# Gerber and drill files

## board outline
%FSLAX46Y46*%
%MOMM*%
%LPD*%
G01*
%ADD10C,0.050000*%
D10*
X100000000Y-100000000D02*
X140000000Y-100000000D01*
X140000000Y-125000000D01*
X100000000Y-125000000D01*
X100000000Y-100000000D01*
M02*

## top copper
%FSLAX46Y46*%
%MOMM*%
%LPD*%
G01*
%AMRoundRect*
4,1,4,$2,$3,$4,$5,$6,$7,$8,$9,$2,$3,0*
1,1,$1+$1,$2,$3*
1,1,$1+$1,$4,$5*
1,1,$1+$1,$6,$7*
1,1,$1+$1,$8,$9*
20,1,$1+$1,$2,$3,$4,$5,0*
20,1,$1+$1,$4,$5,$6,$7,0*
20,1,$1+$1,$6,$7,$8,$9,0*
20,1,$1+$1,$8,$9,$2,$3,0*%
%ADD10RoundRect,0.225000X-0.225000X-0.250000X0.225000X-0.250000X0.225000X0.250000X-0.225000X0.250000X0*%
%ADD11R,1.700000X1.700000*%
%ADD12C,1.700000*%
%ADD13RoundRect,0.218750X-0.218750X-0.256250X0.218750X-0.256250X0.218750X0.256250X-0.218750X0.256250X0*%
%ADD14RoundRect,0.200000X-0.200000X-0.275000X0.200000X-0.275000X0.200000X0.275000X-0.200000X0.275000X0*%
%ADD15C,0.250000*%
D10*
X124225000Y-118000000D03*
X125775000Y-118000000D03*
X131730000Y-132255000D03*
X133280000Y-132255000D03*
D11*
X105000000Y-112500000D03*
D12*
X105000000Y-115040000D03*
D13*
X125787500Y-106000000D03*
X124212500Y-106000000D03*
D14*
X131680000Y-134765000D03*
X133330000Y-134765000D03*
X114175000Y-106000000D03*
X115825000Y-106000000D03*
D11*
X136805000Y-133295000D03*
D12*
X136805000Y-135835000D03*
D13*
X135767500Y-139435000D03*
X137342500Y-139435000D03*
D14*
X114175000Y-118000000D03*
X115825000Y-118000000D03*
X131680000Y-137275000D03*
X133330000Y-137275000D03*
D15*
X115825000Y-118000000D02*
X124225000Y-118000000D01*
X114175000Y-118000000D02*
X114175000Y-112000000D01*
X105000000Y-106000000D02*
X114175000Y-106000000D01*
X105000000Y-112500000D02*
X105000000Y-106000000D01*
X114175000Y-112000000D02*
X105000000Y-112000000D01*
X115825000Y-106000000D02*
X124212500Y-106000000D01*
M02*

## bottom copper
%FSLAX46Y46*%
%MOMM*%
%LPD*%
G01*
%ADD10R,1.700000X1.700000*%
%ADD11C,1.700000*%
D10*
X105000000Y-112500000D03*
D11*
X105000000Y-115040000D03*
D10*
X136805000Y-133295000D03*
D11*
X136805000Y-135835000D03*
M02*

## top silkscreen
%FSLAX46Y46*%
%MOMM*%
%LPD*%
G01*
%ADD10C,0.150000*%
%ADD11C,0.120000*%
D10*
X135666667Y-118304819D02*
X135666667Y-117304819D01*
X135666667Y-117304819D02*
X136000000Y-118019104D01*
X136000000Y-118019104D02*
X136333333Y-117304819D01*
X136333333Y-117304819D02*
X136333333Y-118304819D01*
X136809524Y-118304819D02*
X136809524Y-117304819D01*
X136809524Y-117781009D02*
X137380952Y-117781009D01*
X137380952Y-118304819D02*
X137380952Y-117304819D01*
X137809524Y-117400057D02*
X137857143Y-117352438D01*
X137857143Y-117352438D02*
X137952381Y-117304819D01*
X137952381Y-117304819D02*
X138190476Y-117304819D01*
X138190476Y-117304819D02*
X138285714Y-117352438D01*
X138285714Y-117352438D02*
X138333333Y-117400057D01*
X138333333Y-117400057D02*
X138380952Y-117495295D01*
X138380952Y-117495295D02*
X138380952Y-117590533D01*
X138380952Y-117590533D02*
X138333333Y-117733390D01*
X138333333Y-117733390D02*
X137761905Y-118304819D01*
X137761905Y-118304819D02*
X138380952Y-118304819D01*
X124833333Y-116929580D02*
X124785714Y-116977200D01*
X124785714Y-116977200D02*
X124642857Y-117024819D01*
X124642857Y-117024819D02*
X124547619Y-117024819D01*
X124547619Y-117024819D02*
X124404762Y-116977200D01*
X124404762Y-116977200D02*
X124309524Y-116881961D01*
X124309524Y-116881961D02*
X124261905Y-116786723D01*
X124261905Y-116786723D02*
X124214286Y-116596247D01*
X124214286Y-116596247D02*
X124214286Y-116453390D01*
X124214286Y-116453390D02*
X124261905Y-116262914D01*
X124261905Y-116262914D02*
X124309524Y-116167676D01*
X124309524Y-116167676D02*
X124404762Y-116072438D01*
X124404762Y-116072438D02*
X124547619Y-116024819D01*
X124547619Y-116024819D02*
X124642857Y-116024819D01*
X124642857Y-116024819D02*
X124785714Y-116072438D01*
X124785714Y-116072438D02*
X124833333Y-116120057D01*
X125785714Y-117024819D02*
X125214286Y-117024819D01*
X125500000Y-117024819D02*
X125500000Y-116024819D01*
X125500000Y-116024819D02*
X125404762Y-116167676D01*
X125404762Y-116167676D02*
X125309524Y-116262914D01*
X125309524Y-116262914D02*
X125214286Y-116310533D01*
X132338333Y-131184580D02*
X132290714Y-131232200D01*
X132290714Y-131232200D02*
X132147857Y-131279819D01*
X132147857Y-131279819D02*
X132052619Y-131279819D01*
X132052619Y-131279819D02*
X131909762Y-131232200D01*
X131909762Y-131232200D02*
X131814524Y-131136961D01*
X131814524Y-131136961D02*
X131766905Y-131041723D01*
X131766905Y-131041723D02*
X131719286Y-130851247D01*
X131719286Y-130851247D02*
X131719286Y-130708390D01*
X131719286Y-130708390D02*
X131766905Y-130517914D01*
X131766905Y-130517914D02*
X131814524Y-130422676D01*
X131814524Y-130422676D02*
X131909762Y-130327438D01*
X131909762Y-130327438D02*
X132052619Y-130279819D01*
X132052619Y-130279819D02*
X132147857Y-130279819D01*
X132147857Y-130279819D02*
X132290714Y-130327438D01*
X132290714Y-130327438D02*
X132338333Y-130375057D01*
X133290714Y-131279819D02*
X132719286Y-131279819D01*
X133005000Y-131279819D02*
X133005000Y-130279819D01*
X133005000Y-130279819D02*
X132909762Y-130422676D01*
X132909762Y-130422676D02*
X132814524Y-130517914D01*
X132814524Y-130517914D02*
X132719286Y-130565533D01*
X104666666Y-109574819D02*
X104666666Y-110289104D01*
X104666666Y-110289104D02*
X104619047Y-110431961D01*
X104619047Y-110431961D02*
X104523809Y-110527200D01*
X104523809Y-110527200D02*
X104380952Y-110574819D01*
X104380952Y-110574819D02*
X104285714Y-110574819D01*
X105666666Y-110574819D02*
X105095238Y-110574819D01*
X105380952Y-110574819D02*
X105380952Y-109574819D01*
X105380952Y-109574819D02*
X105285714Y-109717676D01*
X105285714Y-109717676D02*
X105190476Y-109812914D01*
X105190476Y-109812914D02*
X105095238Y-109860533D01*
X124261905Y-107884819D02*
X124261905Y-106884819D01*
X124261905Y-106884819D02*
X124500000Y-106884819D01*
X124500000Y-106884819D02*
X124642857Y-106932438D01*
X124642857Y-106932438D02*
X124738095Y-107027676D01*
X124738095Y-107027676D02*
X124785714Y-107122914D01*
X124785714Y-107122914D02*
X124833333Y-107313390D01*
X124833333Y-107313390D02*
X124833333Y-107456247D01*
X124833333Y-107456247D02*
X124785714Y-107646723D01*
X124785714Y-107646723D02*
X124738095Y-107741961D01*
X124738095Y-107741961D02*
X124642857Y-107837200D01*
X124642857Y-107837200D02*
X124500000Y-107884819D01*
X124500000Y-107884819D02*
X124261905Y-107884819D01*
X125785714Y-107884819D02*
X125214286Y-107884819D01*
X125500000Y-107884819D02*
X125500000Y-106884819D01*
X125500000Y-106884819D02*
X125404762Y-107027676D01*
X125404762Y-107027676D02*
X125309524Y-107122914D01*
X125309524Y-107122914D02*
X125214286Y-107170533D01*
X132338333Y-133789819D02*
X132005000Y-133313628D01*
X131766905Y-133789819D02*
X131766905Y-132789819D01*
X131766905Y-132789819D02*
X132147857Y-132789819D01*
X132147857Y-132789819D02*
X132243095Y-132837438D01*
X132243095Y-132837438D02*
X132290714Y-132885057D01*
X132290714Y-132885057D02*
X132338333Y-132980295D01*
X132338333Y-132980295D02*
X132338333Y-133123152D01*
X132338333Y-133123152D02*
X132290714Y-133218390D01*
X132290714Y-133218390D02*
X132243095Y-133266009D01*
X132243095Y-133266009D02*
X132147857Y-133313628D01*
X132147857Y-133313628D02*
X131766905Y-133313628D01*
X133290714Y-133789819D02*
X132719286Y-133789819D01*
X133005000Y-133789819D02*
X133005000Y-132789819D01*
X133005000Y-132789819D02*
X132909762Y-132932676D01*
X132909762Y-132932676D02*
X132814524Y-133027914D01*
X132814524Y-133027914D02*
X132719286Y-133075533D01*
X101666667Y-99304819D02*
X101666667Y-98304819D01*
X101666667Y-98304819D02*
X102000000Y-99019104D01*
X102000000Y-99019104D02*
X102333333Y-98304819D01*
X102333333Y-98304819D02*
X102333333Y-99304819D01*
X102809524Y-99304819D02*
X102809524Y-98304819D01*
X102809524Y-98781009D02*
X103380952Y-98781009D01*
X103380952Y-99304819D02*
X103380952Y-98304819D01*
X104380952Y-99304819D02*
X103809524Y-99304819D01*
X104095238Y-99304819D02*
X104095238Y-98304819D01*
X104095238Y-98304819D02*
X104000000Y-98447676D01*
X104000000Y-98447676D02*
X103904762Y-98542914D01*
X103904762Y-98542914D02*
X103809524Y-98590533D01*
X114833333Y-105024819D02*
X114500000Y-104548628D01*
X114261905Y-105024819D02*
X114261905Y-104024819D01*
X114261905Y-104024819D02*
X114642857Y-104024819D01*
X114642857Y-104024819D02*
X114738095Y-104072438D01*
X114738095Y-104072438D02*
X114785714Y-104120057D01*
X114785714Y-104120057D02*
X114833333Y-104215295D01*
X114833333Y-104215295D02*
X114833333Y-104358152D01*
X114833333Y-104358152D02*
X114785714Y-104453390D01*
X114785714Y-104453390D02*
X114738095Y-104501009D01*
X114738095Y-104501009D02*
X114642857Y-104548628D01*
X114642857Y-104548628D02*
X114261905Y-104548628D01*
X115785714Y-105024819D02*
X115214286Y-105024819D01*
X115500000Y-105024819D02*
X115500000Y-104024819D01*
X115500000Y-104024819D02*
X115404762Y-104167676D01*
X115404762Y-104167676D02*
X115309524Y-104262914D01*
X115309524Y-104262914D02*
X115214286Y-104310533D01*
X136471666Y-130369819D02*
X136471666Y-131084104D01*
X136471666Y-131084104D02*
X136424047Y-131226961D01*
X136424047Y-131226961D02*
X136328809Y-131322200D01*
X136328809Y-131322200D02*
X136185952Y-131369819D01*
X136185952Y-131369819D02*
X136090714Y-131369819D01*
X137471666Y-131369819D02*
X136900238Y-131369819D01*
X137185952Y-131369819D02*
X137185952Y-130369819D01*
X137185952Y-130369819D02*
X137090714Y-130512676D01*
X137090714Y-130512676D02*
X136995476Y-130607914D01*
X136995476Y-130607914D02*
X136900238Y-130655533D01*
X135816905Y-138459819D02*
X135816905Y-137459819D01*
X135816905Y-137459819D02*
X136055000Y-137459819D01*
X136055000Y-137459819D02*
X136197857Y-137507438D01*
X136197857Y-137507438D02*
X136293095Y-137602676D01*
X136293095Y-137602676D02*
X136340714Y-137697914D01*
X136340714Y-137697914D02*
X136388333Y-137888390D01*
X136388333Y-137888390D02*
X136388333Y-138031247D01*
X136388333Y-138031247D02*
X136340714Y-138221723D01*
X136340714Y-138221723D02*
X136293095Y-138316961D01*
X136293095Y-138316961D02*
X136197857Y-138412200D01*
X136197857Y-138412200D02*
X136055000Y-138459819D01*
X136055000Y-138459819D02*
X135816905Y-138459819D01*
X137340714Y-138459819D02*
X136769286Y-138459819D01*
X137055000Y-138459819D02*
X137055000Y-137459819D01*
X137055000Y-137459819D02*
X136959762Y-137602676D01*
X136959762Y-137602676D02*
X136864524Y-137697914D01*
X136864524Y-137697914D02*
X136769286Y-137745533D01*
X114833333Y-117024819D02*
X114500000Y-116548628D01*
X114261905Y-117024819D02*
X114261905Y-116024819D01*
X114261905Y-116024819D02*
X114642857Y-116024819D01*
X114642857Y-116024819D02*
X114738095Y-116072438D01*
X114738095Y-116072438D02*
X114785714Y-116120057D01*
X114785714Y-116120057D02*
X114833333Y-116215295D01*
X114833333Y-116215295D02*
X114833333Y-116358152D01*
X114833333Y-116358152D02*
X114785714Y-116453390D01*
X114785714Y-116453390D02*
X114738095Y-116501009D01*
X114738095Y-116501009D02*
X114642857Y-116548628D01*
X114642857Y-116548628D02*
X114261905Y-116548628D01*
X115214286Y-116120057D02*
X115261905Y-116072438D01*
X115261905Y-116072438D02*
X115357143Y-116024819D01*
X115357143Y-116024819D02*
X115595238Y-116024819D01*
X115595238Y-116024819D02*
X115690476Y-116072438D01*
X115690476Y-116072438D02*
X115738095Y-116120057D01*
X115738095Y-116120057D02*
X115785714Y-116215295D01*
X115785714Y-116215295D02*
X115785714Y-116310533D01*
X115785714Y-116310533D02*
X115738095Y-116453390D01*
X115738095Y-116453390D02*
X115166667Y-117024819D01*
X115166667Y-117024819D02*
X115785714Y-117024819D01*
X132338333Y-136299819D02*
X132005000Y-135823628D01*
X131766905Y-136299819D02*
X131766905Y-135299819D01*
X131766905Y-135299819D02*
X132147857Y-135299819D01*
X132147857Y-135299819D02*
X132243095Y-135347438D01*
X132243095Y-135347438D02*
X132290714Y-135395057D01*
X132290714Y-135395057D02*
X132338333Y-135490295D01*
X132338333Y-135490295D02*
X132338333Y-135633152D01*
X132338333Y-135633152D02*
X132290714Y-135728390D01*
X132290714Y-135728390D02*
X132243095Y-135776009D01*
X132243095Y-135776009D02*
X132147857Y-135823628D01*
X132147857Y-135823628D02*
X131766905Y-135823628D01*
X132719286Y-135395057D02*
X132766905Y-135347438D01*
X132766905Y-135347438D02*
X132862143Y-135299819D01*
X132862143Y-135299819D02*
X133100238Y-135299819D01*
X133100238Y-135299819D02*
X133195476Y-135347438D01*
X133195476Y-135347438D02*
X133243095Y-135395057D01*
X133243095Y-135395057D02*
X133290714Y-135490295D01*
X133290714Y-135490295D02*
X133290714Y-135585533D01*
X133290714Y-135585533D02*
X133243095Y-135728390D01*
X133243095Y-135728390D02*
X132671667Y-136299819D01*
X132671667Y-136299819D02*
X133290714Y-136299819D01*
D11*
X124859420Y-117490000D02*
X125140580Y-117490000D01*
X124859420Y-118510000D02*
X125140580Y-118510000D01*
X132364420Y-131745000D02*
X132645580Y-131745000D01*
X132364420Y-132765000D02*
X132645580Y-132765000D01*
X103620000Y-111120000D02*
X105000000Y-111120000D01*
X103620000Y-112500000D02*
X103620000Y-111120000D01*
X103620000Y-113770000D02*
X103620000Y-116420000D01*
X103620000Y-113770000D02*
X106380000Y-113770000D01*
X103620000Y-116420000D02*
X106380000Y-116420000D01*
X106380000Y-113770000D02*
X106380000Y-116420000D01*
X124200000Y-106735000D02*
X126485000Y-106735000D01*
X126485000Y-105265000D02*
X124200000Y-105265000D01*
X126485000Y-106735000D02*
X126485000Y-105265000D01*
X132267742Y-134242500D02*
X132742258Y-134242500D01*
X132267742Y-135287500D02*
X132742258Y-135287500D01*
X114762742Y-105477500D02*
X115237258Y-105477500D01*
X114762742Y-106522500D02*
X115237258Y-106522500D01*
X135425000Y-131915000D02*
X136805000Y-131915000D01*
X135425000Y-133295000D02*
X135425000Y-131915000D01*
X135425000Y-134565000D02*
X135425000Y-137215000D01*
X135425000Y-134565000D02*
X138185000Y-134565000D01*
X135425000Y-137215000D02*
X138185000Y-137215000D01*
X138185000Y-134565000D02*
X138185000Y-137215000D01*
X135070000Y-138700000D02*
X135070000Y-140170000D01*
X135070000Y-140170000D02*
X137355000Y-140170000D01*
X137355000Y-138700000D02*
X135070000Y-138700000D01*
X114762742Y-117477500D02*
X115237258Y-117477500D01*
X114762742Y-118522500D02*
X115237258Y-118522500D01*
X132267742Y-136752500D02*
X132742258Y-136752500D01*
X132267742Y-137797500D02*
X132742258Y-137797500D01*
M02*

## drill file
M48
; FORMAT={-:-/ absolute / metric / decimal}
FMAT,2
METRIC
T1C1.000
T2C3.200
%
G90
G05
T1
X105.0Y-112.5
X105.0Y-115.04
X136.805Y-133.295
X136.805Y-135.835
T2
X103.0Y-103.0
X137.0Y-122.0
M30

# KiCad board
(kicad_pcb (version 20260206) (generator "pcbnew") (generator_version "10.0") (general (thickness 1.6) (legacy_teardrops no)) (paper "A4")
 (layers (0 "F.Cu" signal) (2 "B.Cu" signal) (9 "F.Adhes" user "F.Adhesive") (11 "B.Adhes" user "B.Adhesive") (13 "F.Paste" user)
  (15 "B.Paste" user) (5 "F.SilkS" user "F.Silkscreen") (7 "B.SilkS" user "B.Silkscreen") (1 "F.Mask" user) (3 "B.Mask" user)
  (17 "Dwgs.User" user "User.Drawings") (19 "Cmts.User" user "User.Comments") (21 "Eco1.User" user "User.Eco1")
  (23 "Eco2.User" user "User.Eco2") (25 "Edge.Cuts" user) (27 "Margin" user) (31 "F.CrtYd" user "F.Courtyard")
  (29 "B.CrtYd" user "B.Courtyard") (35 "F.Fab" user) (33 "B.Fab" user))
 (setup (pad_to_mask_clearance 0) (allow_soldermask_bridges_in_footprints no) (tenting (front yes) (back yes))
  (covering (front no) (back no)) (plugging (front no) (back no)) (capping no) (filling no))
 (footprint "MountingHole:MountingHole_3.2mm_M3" (layer "F.Cu") (at 137 122)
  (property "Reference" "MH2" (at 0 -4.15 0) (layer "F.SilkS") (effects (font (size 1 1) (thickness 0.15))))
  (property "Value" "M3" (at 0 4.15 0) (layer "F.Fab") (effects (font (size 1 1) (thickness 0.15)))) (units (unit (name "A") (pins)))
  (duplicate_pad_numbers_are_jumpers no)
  (pad "" np_thru_hole circle (at 0 0) (size 3.2 3.2) (drill 3.2) (layers "*.Cu" "*.Mask")))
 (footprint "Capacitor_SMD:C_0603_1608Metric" (layer "F.Cu") (at 125 118)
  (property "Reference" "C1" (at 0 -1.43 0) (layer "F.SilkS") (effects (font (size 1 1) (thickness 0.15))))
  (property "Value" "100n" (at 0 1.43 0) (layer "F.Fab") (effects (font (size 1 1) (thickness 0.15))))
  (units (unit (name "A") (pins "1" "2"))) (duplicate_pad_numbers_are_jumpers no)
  (fp_line (start -0.14058 -0.51) (end 0.14058 -0.51) (stroke (width 0.12) (type solid)) (layer "F.SilkS"))
  (fp_line (start -0.14058 0.51) (end 0.14058 0.51) (stroke (width 0.12) (type solid)) (layer "F.SilkS"))
  (pad "1" smd roundrect (at -0.775 0) (size 0.9 0.95) (layers "F.Cu" "F.Mask" "F.Paste") (roundrect_rratio 0.25) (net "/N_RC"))
  (pad "2" smd roundrect (at 0.775 0) (size 0.9 0.95) (layers "F.Cu" "F.Mask" "F.Paste") (roundrect_rratio 0.25) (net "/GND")))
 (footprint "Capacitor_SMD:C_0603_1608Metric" (layer "F.Cu") (at 132.505 132.255)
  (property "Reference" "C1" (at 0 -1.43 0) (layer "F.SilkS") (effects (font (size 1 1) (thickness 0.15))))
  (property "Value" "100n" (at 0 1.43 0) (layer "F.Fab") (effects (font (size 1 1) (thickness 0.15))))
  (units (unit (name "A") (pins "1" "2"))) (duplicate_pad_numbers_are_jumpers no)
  (fp_line (start -0.14058 -0.51) (end 0.14058 -0.51) (stroke (width 0.12) (type solid)) (layer "F.SilkS"))
  (fp_line (start -0.14058 0.51) (end 0.14058 0.51) (stroke (width 0.12) (type solid)) (layer "F.SilkS"))
  (pad "1" smd roundrect (at -0.775 0) (size 0.9 0.95) (layers "F.Cu" "F.Mask" "F.Paste") (roundrect_rratio 0.25) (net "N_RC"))
  (pad "2" smd roundrect (at 0.775 0) (size 0.9 0.95) (layers "F.Cu" "F.Mask" "F.Paste") (roundrect_rratio 0.25) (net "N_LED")))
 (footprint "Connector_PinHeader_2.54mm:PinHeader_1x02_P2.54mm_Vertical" (layer "F.Cu") (at 105 112.5)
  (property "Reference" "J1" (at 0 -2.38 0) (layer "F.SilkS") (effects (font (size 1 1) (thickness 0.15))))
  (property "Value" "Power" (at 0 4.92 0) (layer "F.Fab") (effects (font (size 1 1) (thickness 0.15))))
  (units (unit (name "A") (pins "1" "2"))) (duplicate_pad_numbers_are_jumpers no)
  (fp_line (start -1.38 -1.38) (end 0 -1.38) (stroke (width 0.12) (type solid)) (layer "F.SilkS"))
  (fp_line (start -1.38 0) (end -1.38 -1.38) (stroke (width 0.12) (type solid)) (layer "F.SilkS"))
  (fp_line (start -1.38 1.27) (end -1.38 3.92) (stroke (width 0.12) (type solid)) (layer "F.SilkS"))
  (fp_line (start -1.38 1.27) (end 1.38 1.27) (stroke (width 0.12) (type solid)) (layer "F.SilkS"))
  (fp_line (start -1.38 3.92) (end 1.38 3.92) (stroke (width 0.12) (type solid)) (layer "F.SilkS"))
  (fp_line (start 1.38 1.27) (end 1.38 3.92) (stroke (width 0.12) (type solid)) (layer "F.SilkS"))
  (pad "1" thru_hole rect (at 0 0) (size 1.7 1.7) (drill 1) (layers "*.Cu" "*.Mask") (remove_unused_layers no) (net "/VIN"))
  (pad "2" thru_hole circle (at 0 2.54) (size 1.7 1.7) (drill 1) (layers "*.Cu" "*.Mask") (remove_unused_layers no) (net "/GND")))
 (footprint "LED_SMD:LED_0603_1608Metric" (layer "F.Cu") (at 125 106 180)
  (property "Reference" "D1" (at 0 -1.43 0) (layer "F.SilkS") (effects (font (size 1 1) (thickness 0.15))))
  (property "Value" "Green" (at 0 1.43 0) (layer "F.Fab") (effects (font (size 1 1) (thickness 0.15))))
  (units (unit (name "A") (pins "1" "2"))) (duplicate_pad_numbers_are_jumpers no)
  (fp_line (start 0.8 -0.735) (end -1.485 -0.735) (stroke (width 0.12) (type solid)) (layer "F.SilkS"))
  (fp_line (start -1.485 0.735) (end 0.8 0.735) (stroke (width 0.12) (type solid)) (layer "F.SilkS"))
  (fp_line (start -1.485 -0.735) (end -1.485 0.735) (stroke (width 0.12) (type solid)) (layer "F.SilkS"))
  (pad "1" smd roundrect (at -0.7875 0) (size 0.875 0.95) (layers "F.Cu" "F.Mask" "F.Paste") (roundrect_rratio 0.25) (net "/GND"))
  (pad "2" smd roundrect (at 0.7875 0) (size 0.875 0.95) (layers "F.Cu" "F.Mask" "F.Paste") (roundrect_rratio 0.25) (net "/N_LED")))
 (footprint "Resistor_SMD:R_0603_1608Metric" (layer "F.Cu") (at 132.505 134.765)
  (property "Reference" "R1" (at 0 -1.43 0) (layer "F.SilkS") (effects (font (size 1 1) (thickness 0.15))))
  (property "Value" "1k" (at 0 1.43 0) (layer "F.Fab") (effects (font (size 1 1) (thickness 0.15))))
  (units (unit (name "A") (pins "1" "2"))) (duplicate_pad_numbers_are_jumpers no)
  (fp_line (start -0.237258 -0.5225) (end 0.237258 -0.5225) (stroke (width 0.12) (type solid)) (layer "F.SilkS"))
  (fp_line (start -0.237258 0.5225) (end 0.237258 0.5225) (stroke (width 0.12) (type solid)) (layer "F.SilkS"))
  (pad "1" smd roundrect (at -0.825 0) (size 0.8 0.95) (layers "F.Cu" "F.Mask" "F.Paste") (roundrect_rratio 0.25) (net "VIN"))
  (pad "2" smd roundrect (at 0.825 0) (size 0.8 0.95) (layers "F.Cu" "F.Mask" "F.Paste") (roundrect_rratio 0.25) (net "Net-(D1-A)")))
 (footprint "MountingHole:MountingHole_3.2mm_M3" (layer "F.Cu") (at 103 103)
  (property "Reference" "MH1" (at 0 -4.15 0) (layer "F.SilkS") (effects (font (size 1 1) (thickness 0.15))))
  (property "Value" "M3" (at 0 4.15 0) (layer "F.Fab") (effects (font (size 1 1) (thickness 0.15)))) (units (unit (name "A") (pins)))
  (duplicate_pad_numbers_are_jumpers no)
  (pad "" np_thru_hole circle (at 0 0) (size 3.2 3.2) (drill 3.2) (layers "*.Cu" "*.Mask")))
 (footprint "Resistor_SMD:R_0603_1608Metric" (layer "F.Cu") (at 115 106)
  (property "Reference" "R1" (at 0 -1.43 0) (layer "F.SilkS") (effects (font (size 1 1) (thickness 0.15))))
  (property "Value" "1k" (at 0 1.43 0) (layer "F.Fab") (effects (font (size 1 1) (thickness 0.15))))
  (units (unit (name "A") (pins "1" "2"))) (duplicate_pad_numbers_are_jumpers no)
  (fp_line (start -0.237258 -0.5225) (end 0.237258 -0.5225) (stroke (width 0.12) (type solid)) (layer "F.SilkS"))
  (fp_line (start -0.237258 0.5225) (end 0.237258 0.5225) (stroke (width 0.12) (type solid)) (layer "F.SilkS"))
  (pad "1" smd roundrect (at -0.825 0) (size 0.8 0.95) (layers "F.Cu" "F.Mask" "F.Paste") (roundrect_rratio 0.25) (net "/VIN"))
  (pad "2" smd roundrect (at 0.825 0) (size 0.8 0.95) (layers "F.Cu" "F.Mask" "F.Paste") (roundrect_rratio 0.25) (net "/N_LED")))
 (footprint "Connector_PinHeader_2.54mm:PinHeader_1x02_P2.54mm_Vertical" (layer "F.Cu") (at 136.805 133.295)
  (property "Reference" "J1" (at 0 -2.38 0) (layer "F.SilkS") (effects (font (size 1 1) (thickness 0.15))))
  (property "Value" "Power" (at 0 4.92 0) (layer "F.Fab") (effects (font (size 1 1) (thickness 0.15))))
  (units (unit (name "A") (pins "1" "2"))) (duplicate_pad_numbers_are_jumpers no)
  (fp_line (start -1.38 -1.38) (end 0 -1.38) (stroke (width 0.12) (type solid)) (layer "F.SilkS"))
  (fp_line (start -1.38 0) (end -1.38 -1.38) (stroke (width 0.12) (type solid)) (layer "F.SilkS"))
  (fp_line (start -1.38 1.27) (end -1.38 3.92) (stroke (width 0.12) (type solid)) (layer "F.SilkS"))
  (fp_line (start -1.38 1.27) (end 1.38 1.27) (stroke (width 0.12) (type solid)) (layer "F.SilkS"))
  (fp_line (start -1.38 3.92) (end 1.38 3.92) (stroke (width 0.12) (type solid)) (layer "F.SilkS"))
  (fp_line (start 1.38 1.27) (end 1.38 3.92) (stroke (width 0.12) (type solid)) (layer "F.SilkS"))
  (pad "1" thru_hole rect (at 0 0) (size 1.7 1.7) (drill 1) (layers "*.Cu" "*.Mask") (remove_unused_layers no) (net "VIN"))
  (pad "2" thru_hole circle (at 0 2.54) (size 1.7 1.7) (drill 1) (layers "*.Cu" "*.Mask") (remove_unused_layers no) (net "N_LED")))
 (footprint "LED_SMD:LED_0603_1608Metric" (layer "F.Cu") (at 136.555 139.435)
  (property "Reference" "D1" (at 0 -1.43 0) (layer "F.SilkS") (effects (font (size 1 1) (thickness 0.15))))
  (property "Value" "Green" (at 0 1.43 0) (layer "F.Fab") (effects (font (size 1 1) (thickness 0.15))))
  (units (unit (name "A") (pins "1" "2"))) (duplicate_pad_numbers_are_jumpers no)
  (fp_line (start -1.485 -0.735) (end -1.485 0.735) (stroke (width 0.12) (type solid)) (layer "F.SilkS"))
  (fp_line (start -1.485 0.735) (end 0.8 0.735) (stroke (width 0.12) (type solid)) (layer "F.SilkS"))
  (fp_line (start 0.8 -0.735) (end -1.485 -0.735) (stroke (width 0.12) (type solid)) (layer "F.SilkS"))
  (pad "1" smd roundrect (at -0.7875 0) (size 0.875 0.95) (layers "F.Cu" "F.Mask" "F.Paste") (roundrect_rratio 0.25) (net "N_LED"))
  (pad "2" smd roundrect (at 0.7875 0) (size 0.875 0.95) (layers "F.Cu" "F.Mask" "F.Paste") (roundrect_rratio 0.25) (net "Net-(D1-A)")))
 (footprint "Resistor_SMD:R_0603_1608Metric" (layer "F.Cu") (at 115 118)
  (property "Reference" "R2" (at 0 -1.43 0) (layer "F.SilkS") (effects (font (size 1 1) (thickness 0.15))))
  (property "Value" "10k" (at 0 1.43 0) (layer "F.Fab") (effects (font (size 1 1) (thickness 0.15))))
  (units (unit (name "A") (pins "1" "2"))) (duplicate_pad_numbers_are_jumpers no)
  (fp_line (start -0.237258 -0.5225) (end 0.237258 -0.5225) (stroke (width 0.12) (type solid)) (layer "F.SilkS"))
  (fp_line (start -0.237258 0.5225) (end 0.237258 0.5225) (stroke (width 0.12) (type solid)) (layer "F.SilkS"))
  (pad "1" smd roundrect (at -0.825 0) (size 0.8 0.95) (layers "F.Cu" "F.Mask" "F.Paste") (roundrect_rratio 0.25) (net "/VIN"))
  (pad "2" smd roundrect (at 0.825 0) (size 0.8 0.95) (layers "F.Cu" "F.Mask" "F.Paste") (roundrect_rratio 0.25) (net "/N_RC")))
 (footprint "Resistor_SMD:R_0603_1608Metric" (layer "F.Cu") (at 132.505 137.275)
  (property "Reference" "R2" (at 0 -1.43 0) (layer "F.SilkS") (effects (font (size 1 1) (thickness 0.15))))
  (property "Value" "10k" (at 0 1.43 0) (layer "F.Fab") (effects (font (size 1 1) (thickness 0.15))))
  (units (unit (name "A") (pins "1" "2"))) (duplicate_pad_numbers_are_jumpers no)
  (fp_line (start -0.237258 -0.5225) (end 0.237258 -0.5225) (stroke (width 0.12) (type solid)) (layer "F.SilkS"))
  (fp_line (start -0.237258 0.5225) (end 0.237258 0.5225) (stroke (width 0.12) (type solid)) (layer "F.SilkS"))
  (pad "1" smd roundrect (at -0.825 0) (size 0.8 0.95) (layers "F.Cu" "F.Mask" "F.Paste") (roundrect_rratio 0.25) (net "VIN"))
  (pad "2" smd roundrect (at 0.825 0) (size 0.8 0.95) (layers "F.Cu" "F.Mask" "F.Paste") (roundrect_rratio 0.25)
   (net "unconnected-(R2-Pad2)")))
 (gr_rect (start 100 100) (end 140 125) (stroke (width 0.05) (type default)) (fill no) (layer "Edge.Cuts"))
 (segment (start 115.825 118) (end 124.225 118) (width 0.25) (layer "F.Cu") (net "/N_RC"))
 (segment (start 114.175 118) (end 114.175 112) (width 0.25) (layer "F.Cu") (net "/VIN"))
 (segment (start 105 106) (end 114.175 106) (width 0.25) (layer "F.Cu") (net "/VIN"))
 (segment (start 105 112.5) (end 105 106) (width 0.25) (layer "F.Cu") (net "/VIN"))
 (segment (start 114.175 112) (end 105 112) (width 0.25) (layer "F.Cu") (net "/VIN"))
 (segment (start 115.825 106) (end 124.2125 106) (width 0.25) (layer "F.Cu") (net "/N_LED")))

